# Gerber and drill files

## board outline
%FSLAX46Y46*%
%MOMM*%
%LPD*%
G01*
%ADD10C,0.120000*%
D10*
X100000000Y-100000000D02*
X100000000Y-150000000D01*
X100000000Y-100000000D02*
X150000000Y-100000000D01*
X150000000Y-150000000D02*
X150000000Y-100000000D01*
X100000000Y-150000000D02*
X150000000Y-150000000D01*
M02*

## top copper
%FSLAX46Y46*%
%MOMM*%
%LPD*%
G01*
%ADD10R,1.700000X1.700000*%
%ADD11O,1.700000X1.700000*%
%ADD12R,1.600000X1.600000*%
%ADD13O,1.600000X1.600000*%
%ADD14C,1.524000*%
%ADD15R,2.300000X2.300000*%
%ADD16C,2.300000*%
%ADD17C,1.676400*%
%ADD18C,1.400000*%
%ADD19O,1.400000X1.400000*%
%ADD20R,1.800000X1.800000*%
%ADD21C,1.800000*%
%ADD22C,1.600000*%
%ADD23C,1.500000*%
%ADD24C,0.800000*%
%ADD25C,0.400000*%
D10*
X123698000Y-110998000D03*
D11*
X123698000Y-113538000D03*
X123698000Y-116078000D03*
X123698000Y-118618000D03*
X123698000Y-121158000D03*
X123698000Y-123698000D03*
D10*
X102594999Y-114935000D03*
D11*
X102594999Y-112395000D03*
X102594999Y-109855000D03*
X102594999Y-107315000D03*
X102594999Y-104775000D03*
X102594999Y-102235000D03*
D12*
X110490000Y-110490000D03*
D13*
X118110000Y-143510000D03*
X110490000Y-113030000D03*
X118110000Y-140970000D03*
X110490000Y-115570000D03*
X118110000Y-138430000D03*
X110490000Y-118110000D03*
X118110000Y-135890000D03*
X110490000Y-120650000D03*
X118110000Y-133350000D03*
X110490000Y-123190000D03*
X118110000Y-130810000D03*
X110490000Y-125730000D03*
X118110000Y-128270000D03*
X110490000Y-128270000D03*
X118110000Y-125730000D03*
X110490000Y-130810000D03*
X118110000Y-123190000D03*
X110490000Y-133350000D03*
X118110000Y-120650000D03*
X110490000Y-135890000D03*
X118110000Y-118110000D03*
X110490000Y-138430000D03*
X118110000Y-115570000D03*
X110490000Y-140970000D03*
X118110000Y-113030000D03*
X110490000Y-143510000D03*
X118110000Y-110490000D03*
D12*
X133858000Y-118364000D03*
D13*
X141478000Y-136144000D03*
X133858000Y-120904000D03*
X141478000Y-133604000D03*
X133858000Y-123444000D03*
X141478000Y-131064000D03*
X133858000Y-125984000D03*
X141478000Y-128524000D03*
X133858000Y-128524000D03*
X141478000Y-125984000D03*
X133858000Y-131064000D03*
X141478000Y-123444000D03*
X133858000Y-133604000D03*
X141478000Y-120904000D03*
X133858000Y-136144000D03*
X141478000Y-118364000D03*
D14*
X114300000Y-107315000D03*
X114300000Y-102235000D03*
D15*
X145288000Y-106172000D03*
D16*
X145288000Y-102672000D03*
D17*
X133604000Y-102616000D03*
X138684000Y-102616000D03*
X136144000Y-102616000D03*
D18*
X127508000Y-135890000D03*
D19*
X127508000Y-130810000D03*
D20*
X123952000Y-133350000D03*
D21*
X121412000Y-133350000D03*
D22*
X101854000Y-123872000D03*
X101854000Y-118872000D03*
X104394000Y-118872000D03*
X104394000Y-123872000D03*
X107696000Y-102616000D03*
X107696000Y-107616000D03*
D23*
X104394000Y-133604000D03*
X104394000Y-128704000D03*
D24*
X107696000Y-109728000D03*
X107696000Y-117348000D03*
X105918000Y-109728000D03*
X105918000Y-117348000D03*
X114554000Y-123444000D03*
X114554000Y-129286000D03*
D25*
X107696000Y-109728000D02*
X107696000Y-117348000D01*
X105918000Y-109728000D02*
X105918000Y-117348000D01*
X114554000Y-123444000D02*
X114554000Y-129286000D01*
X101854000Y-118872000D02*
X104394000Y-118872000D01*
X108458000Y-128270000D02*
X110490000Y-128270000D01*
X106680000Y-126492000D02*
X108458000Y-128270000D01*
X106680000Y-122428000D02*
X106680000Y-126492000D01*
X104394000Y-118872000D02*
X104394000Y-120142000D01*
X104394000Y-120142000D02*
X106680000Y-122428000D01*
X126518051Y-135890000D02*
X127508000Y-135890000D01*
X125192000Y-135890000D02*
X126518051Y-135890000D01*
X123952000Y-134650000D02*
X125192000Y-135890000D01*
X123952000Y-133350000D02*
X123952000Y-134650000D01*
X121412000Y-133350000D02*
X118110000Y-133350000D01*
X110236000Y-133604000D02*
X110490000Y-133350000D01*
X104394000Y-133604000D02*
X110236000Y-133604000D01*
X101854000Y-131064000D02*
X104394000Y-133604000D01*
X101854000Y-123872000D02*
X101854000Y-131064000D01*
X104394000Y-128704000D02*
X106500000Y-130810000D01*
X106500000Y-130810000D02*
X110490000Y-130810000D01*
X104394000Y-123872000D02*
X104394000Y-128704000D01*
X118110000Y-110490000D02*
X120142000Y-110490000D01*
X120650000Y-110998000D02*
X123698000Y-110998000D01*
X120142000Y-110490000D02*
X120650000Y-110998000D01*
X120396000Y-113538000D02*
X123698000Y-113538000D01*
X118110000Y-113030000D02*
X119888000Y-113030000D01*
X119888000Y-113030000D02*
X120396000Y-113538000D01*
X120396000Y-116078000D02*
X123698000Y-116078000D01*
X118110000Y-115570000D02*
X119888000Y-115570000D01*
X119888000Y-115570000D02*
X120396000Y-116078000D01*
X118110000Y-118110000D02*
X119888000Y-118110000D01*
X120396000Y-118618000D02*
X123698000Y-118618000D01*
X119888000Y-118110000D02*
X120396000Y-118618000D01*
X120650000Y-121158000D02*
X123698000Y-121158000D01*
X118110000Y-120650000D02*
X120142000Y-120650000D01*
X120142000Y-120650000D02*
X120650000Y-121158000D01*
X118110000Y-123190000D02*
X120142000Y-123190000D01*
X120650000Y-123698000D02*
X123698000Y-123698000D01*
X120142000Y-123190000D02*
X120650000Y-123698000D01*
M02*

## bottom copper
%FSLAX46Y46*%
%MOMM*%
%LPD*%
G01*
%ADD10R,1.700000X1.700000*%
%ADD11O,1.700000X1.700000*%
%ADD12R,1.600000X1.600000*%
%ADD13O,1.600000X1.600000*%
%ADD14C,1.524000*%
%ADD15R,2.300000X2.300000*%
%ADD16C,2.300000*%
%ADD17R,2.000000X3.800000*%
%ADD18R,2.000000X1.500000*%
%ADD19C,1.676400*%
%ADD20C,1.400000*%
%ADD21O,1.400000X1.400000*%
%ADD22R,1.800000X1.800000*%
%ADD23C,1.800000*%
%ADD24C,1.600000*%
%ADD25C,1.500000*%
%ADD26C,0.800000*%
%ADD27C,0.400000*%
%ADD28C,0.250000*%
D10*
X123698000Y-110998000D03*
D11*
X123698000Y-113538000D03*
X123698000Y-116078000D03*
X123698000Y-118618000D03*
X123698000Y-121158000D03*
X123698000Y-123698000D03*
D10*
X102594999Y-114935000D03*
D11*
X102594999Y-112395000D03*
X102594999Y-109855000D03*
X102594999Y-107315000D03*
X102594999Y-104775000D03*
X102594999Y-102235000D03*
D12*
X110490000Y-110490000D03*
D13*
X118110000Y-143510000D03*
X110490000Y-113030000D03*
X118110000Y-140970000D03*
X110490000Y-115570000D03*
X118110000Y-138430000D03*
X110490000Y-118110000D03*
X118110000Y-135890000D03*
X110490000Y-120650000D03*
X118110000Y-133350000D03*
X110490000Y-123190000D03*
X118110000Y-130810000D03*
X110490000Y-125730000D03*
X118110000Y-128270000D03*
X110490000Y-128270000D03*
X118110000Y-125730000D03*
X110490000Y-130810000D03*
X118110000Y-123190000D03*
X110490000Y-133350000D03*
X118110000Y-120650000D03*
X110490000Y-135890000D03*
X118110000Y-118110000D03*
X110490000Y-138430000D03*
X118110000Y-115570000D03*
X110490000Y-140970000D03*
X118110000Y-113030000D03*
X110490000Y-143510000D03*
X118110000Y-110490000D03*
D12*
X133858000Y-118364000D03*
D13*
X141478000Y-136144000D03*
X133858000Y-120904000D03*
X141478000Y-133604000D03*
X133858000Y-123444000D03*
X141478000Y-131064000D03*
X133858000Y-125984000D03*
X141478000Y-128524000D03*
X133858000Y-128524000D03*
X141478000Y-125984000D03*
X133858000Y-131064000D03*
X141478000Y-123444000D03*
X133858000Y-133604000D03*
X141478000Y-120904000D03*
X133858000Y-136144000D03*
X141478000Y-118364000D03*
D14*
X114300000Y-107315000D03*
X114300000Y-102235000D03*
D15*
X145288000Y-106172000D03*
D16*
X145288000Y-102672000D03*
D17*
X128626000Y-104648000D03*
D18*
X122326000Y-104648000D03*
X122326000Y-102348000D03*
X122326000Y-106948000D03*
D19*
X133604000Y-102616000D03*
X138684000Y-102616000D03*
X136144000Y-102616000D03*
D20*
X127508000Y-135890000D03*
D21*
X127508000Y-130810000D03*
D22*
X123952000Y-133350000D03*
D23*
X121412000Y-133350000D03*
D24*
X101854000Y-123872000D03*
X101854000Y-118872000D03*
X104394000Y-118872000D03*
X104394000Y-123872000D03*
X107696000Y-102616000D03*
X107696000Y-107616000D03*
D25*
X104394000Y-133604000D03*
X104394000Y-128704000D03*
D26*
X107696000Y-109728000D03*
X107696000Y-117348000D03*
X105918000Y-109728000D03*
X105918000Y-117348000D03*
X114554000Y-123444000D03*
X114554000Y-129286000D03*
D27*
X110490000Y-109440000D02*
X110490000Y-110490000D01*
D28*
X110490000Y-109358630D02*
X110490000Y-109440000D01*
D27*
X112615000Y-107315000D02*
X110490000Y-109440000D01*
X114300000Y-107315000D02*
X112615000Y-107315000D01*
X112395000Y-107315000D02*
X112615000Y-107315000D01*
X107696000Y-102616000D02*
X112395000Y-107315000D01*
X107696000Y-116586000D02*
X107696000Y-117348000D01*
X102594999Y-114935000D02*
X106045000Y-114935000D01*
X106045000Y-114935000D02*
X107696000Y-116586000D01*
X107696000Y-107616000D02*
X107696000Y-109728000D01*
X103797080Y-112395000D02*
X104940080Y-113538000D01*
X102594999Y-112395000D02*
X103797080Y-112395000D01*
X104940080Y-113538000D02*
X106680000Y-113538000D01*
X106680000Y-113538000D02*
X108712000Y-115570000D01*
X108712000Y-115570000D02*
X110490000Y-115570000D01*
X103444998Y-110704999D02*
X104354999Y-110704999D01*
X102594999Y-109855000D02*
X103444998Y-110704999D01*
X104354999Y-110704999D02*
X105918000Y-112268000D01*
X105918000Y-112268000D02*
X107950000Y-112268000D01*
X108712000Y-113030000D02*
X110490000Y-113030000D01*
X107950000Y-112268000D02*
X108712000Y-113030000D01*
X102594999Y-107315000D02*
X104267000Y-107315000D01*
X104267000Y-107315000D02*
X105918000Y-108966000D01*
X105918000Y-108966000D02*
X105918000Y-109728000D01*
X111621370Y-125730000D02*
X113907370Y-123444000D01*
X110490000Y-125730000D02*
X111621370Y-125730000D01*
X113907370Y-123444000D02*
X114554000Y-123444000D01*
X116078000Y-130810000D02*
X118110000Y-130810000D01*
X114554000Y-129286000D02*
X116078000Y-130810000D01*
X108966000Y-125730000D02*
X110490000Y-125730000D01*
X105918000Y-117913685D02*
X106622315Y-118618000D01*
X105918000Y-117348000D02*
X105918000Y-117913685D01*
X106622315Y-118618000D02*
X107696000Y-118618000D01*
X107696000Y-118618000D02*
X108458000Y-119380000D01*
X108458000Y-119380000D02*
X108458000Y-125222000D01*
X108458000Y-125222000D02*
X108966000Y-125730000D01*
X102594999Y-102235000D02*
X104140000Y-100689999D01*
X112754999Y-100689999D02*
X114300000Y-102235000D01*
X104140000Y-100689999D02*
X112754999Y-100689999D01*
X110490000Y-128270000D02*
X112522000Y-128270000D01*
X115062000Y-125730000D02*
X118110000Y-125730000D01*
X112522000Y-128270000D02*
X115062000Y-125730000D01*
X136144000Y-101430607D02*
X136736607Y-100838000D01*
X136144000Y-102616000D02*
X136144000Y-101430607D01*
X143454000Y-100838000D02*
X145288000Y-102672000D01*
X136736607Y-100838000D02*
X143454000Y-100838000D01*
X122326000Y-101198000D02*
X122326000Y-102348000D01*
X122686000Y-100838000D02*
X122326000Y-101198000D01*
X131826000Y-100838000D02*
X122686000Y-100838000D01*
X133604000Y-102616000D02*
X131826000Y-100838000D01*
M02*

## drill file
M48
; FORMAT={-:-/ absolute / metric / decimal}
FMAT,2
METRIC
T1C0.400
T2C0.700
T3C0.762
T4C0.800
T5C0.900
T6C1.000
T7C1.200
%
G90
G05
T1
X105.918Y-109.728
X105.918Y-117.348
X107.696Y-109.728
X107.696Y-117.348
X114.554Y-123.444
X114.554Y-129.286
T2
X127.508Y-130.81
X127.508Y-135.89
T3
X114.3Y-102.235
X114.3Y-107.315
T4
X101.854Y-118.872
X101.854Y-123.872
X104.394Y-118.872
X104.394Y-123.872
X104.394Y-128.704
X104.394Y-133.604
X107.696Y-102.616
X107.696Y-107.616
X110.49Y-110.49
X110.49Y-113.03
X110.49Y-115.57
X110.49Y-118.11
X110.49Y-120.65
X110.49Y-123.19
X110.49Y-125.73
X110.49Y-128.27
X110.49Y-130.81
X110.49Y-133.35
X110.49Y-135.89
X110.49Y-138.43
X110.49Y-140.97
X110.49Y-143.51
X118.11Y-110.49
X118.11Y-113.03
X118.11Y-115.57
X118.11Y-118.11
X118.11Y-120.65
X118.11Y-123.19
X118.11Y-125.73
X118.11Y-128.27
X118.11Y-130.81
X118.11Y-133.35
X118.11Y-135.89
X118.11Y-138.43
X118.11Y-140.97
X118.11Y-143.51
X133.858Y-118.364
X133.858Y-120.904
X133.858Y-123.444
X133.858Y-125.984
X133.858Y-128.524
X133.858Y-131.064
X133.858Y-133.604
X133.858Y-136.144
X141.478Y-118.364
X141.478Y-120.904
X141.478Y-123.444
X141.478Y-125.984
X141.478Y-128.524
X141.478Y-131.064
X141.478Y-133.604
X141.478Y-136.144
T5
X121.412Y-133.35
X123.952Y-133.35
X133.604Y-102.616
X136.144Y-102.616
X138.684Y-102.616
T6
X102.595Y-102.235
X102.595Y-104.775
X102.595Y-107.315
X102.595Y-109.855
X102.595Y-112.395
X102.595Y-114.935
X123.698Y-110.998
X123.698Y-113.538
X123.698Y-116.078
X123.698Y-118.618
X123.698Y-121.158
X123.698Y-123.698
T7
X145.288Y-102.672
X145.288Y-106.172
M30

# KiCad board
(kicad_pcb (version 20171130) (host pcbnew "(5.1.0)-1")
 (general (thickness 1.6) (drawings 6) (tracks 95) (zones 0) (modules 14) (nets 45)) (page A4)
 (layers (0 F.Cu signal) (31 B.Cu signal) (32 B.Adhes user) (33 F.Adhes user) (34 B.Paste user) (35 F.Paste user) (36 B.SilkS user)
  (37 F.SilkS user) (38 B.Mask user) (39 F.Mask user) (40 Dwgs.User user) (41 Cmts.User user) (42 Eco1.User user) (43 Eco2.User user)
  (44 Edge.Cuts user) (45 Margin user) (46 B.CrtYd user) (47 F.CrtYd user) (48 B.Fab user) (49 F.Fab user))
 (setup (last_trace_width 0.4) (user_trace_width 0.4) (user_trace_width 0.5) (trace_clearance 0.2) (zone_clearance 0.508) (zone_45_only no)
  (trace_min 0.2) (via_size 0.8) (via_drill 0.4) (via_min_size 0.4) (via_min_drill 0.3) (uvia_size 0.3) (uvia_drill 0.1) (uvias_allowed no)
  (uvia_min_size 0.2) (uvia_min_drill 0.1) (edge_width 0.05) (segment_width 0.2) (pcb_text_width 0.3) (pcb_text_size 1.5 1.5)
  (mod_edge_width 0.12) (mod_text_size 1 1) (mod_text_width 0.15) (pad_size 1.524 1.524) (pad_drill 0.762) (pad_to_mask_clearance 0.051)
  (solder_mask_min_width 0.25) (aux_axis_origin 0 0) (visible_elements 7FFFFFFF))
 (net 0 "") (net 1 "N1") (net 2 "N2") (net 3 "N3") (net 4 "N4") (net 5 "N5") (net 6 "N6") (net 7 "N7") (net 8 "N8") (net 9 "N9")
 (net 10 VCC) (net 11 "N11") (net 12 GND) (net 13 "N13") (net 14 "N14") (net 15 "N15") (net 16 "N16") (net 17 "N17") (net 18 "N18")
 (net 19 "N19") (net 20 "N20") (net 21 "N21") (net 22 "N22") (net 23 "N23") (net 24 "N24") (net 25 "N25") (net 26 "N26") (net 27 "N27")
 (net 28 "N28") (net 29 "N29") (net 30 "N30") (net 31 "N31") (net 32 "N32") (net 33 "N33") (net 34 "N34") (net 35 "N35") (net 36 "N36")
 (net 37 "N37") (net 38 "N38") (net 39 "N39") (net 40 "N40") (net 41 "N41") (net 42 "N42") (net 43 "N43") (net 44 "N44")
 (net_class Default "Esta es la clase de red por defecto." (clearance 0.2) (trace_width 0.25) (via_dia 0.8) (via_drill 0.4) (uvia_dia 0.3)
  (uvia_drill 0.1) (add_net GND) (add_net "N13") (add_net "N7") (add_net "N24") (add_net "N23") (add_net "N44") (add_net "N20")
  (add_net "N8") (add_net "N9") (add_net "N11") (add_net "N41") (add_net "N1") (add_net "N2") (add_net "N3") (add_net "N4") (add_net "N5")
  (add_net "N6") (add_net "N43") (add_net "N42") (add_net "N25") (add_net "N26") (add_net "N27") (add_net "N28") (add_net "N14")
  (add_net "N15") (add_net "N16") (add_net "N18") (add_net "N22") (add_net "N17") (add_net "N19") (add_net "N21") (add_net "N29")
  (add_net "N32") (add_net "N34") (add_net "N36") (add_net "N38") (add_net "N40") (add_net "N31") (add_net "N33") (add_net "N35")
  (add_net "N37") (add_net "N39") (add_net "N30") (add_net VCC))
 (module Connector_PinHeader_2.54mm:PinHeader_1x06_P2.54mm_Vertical (layer F.Cu) (at 123.698 110.998)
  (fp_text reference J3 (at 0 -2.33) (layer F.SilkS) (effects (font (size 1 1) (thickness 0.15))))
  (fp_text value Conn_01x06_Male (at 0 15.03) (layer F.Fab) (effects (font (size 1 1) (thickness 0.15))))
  (pad 1 thru_hole rect (at 0 0) (size 1.7 1.7) (drill 1) (layers *.Cu *.Mask) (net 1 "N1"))
  (pad 2 thru_hole oval (at 0 2.54) (size 1.7 1.7) (drill 1) (layers *.Cu *.Mask) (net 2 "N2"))
  (pad 3 thru_hole oval (at 0 5.08) (size 1.7 1.7) (drill 1) (layers *.Cu *.Mask) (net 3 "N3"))
  (pad 4 thru_hole oval (at 0 7.62) (size 1.7 1.7) (drill 1) (layers *.Cu *.Mask) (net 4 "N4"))
  (pad 5 thru_hole oval (at 0 10.16) (size 1.7 1.7) (drill 1) (layers *.Cu *.Mask) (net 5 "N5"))
  (pad 6 thru_hole oval (at 0 12.7) (size 1.7 1.7) (drill 1) (layers *.Cu *.Mask) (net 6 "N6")))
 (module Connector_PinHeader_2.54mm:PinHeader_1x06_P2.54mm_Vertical (layer F.Cu) (at 102.594999 114.935 180)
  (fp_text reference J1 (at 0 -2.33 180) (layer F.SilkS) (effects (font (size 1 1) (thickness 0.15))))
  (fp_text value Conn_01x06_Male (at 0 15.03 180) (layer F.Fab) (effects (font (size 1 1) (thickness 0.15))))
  (pad 1 thru_hole rect (at 0 0 180) (size 1.7 1.7) (drill 1) (layers *.Cu *.Mask) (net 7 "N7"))
  (pad 2 thru_hole oval (at 0 2.54 180) (size 1.7 1.7) (drill 1) (layers *.Cu *.Mask) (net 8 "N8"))
  (pad 3 thru_hole oval (at 0 5.08 180) (size 1.7 1.7) (drill 1) (layers *.Cu *.Mask) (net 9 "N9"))
  (pad 4 thru_hole oval (at 0 7.62 180) (size 1.7 1.7) (drill 1) (layers *.Cu *.Mask) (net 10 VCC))
  (pad 5 thru_hole oval (at 0 10.16 180) (size 1.7 1.7) (drill 1) (layers *.Cu *.Mask) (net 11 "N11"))
  (pad 6 thru_hole oval (at 0 12.7 180) (size 1.7 1.7) (drill 1) (layers *.Cu *.Mask) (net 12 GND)))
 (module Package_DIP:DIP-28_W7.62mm (layer F.Cu) (at 110.49 110.49)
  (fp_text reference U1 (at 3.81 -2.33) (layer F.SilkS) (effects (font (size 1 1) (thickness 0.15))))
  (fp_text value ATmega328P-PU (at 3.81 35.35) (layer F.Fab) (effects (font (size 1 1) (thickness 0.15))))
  (pad 1 thru_hole rect (at 0 0) (size 1.6 1.6) (drill 0.8) (layers *.Cu *.Mask) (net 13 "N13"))
  (pad 15 thru_hole oval (at 7.62 33.02) (size 1.6 1.6) (drill 0.8) (layers *.Cu *.Mask) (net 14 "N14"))
  (pad 2 thru_hole oval (at 0 2.54) (size 1.6 1.6) (drill 0.8) (layers *.Cu *.Mask) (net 9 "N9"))
  (pad 16 thru_hole oval (at 7.62 30.48) (size 1.6 1.6) (drill 0.8) (layers *.Cu *.Mask) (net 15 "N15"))
  (pad 3 thru_hole oval (at 0 5.08) (size 1.6 1.6) (drill 0.8) (layers *.Cu *.Mask) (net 8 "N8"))
  (pad 17 thru_hole oval (at 7.62 27.94) (size 1.6 1.6) (drill 0.8) (layers *.Cu *.Mask) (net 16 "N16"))
  (pad 4 thru_hole oval (at 0 7.62) (size 1.6 1.6) (drill 0.8) (layers *.Cu *.Mask) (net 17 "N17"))
  (pad 18 thru_hole oval (at 7.62 25.4) (size 1.6 1.6) (drill 0.8) (layers *.Cu *.Mask) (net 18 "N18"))
  (pad 5 thru_hole oval (at 0 10.16) (size 1.6 1.6) (drill 0.8) (layers *.Cu *.Mask) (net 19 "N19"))
  (pad 19 thru_hole oval (at 7.62 22.86) (size 1.6 1.6) (drill 0.8) (layers *.Cu *.Mask) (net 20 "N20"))
  (pad 6 thru_hole oval (at 0 12.7) (size 1.6 1.6) (drill 0.8) (layers *.Cu *.Mask) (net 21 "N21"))
  (pad 20 thru_hole oval (at 7.62 20.32) (size 1.6 1.6) (drill 0.8) (layers *.Cu *.Mask) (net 10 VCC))
  (pad 7 thru_hole oval (at 0 15.24) (size 1.6 1.6) (drill 0.8) (layers *.Cu *.Mask) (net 10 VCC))
  (pad 21 thru_hole oval (at 7.62 17.78) (size 1.6 1.6) (drill 0.8) (layers *.Cu *.Mask) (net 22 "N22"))
  (pad 8 thru_hole oval (at 0 17.78) (size 1.6 1.6) (drill 0.8) (layers *.Cu *.Mask) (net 12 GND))
  (pad 22 thru_hole oval (at 7.62 15.24) (size 1.6 1.6) (drill 0.8) (layers *.Cu *.Mask) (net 12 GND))
  (pad 9 thru_hole oval (at 0 20.32) (size 1.6 1.6) (drill 0.8) (layers *.Cu *.Mask) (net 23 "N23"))
  (pad 23 thru_hole oval (at 7.62 12.7) (size 1.6 1.6) (drill 0.8) (layers *.Cu *.Mask) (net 6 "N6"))
  (pad 10 thru_hole oval (at 0 22.86) (size 1.6 1.6) (drill 0.8) (layers *.Cu *.Mask) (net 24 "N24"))
  (pad 24 thru_hole oval (at 7.62 10.16) (size 1.6 1.6) (drill 0.8) (layers *.Cu *.Mask) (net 5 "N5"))
  (pad 11 thru_hole oval (at 0 25.4) (size 1.6 1.6) (drill 0.8) (layers *.Cu *.Mask) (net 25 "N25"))
  (pad 25 thru_hole oval (at 7.62 7.62) (size 1.6 1.6) (drill 0.8) (layers *.Cu *.Mask) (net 4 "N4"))
  (pad 12 thru_hole oval (at 0 27.94) (size 1.6 1.6) (drill 0.8) (layers *.Cu *.Mask) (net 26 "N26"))
  (pad 26 thru_hole oval (at 7.62 5.08) (size 1.6 1.6) (drill 0.8) (layers *.Cu *.Mask) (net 3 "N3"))
  (pad 13 thru_hole oval (at 0 30.48) (size 1.6 1.6) (drill 0.8) (layers *.Cu *.Mask) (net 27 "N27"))
  (pad 27 thru_hole oval (at 7.62 2.54) (size 1.6 1.6) (drill 0.8) (layers *.Cu *.Mask) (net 2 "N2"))
  (pad 14 thru_hole oval (at 0 33.02) (size 1.6 1.6) (drill 0.8) (layers *.Cu *.Mask) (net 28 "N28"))
  (pad 28 thru_hole oval (at 7.62 0) (size 1.6 1.6) (drill 0.8) (layers *.Cu *.Mask) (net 1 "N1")))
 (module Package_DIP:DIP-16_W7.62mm (layer F.Cu) (at 133.858 118.364)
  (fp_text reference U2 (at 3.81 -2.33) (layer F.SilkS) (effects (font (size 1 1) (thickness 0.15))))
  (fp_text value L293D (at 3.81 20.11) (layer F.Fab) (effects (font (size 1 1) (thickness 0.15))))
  (pad 1 thru_hole rect (at 0 0) (size 1.6 1.6) (drill 0.8) (layers *.Cu *.Mask) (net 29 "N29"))
  (pad 9 thru_hole oval (at 7.62 17.78) (size 1.6 1.6) (drill 0.8) (layers *.Cu *.Mask) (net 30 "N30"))
  (pad 2 thru_hole oval (at 0 2.54) (size 1.6 1.6) (drill 0.8) (layers *.Cu *.Mask) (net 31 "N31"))
  (pad 10 thru_hole oval (at 7.62 15.24) (size 1.6 1.6) (drill 0.8) (layers *.Cu *.Mask) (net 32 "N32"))
  (pad 3 thru_hole oval (at 0 5.08) (size 1.6 1.6) (drill 0.8) (layers *.Cu *.Mask) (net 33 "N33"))
  (pad 11 thru_hole oval (at 7.62 12.7) (size 1.6 1.6) (drill 0.8) (layers *.Cu *.Mask) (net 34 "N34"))
  (pad 4 thru_hole oval (at 0 7.62) (size 1.6 1.6) (drill 0.8) (layers *.Cu *.Mask) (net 12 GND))
  (pad 12 thru_hole oval (at 7.62 10.16) (size 1.6 1.6) (drill 0.8) (layers *.Cu *.Mask) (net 12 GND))
  (pad 5 thru_hole oval (at 0 10.16) (size 1.6 1.6) (drill 0.8) (layers *.Cu *.Mask) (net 12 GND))
  (pad 13 thru_hole oval (at 7.62 7.62) (size 1.6 1.6) (drill 0.8) (layers *.Cu *.Mask) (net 12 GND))
  (pad 6 thru_hole oval (at 0 12.7) (size 1.6 1.6) (drill 0.8) (layers *.Cu *.Mask) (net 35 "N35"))
  (pad 14 thru_hole oval (at 7.62 5.08) (size 1.6 1.6) (drill 0.8) (layers *.Cu *.Mask) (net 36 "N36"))
  (pad 7 thru_hole oval (at 0 15.24) (size 1.6 1.6) (drill 0.8) (layers *.Cu *.Mask) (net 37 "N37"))
  (pad 15 thru_hole oval (at 7.62 2.54) (size 1.6 1.6) (drill 0.8) (layers *.Cu *.Mask) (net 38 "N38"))
  (pad 8 thru_hole oval (at 0 17.78) (size 1.6 1.6) (drill 0.8) (layers *.Cu *.Mask) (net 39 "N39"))
  (pad 16 thru_hole oval (at 7.62 0) (size 1.6 1.6) (drill 0.8) (layers *.Cu *.Mask) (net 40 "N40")))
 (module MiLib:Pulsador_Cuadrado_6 (layer F.Cu) (at 111.76 104.775 90)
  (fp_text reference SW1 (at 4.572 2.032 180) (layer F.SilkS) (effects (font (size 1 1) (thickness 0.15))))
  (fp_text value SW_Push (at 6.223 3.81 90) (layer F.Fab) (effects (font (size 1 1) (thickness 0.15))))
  (pad 1 thru_hole circle (at -2.54 2.54 90) (size 1.524 1.524) (drill 0.762) (layers *.Cu *.Mask) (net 13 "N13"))
  (pad 2 thru_hole circle (at 2.54 2.54 90) (size 1.524 1.524) (drill 0.762) (layers *.Cu *.Mask) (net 12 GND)))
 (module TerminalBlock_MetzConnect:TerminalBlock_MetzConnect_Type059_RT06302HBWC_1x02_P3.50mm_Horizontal (layer F.Cu)
  (at 145.288 106.172 90)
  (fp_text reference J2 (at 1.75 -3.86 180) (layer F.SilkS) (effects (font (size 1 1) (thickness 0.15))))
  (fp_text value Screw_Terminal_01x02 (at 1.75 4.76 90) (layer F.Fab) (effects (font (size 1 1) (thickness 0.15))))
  (pad 1 thru_hole rect (at 0 0 90) (size 2.3 2.3) (drill 1.2) (layers *.Cu *.Mask) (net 12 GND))
  (pad 2 thru_hole circle (at 3.5 0 90) (size 2.3 2.3) (drill 1.2) (layers *.Cu *.Mask) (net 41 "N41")))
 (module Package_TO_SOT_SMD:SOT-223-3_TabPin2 (layer B.Cu) (at 125.476 104.648)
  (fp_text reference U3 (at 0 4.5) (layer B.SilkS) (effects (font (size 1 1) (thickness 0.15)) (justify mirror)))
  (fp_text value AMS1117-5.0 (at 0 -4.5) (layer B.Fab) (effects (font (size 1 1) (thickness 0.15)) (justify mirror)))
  (pad 2 smd rect (at 3.15 0) (size 2 3.8) (layers B.Cu B.Paste B.Mask) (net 10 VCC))
  (pad 2 smd rect (at -3.15 0) (size 2 1.5) (layers B.Cu B.Paste B.Mask) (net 10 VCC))
  (pad 3 smd rect (at -3.15 -2.3) (size 2 1.5) (layers B.Cu B.Paste B.Mask) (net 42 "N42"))
  (pad 1 smd rect (at -3.15 2.3) (size 2 1.5) (layers B.Cu B.Paste B.Mask) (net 12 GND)))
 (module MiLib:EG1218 (layer F.Cu) (at 136.144 102.616 180)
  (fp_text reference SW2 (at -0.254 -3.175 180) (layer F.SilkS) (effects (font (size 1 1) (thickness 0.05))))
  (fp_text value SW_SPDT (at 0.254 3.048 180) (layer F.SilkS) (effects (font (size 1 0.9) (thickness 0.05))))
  (pad 3 thru_hole circle (at 2.54 0 180) (size 1.6764 1.6764) (drill 0.9) (layers *.Cu *.Mask) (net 42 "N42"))
  (pad 1 thru_hole circle (at -2.54 0 180) (size 1.6764 1.6764) (drill 0.9) (layers *.Cu *.Mask) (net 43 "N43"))
  (pad 2 thru_hole circle (at 0 0 180) (size 1.6764 1.6764) (drill 0.9) (layers *.Cu *.Mask) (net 41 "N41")))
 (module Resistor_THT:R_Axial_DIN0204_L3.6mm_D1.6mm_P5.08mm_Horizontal (layer F.Cu) (at 127.508 135.89 90)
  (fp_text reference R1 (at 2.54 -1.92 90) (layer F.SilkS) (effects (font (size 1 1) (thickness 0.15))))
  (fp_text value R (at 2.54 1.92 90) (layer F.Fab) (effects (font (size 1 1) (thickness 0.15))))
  (pad 1 thru_hole circle (at 0 0 90) (size 1.4 1.4) (drill 0.7) (layers *.Cu *.Mask) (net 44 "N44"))
  (pad 2 thru_hole oval (at 5.08 0 90) (size 1.4 1.4) (drill 0.7) (layers *.Cu *.Mask) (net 12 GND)))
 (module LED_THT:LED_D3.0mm (layer F.Cu) (at 123.952 133.35 180)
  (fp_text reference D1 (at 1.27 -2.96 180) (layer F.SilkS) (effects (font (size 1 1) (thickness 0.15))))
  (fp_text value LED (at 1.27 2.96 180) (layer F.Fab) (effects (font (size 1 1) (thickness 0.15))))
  (pad 1 thru_hole rect (at 0 0 180) (size 1.8 1.8) (drill 0.9) (layers *.Cu *.Mask) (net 44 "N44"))
  (pad 2 thru_hole circle (at 2.54 0 180) (size 1.8 1.8) (drill 0.9) (layers *.Cu *.Mask) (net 20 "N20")))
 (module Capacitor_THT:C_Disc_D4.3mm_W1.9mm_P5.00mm (layer F.Cu) (at 101.854 123.872 90)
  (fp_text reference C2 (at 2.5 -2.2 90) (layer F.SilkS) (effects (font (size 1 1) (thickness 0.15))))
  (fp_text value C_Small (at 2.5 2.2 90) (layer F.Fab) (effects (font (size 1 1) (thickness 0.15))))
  (pad 1 thru_hole circle (at 0 0 90) (size 1.6 1.6) (drill 0.8) (layers *.Cu *.Mask) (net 24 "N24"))
  (pad 2 thru_hole circle (at 5 0 90) (size 1.6 1.6) (drill 0.8) (layers *.Cu *.Mask) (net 12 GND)))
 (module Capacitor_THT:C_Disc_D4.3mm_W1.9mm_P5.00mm (layer F.Cu) (at 104.394 123.872 90)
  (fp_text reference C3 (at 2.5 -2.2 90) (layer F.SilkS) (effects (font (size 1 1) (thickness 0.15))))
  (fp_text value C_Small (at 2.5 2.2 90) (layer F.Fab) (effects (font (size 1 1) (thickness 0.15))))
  (pad 2 thru_hole circle (at 5 0 90) (size 1.6 1.6) (drill 0.8) (layers *.Cu *.Mask) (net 12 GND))
  (pad 1 thru_hole circle (at 0 0 90) (size 1.6 1.6) (drill 0.8) (layers *.Cu *.Mask) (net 23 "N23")))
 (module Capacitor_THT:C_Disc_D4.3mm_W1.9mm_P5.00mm (layer F.Cu) (at 107.696 102.616 270)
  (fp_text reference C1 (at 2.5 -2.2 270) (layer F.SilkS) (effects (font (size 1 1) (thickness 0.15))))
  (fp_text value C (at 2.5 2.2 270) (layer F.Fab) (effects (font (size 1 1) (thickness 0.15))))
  (pad 1 thru_hole circle (at 0 0 270) (size 1.6 1.6) (drill 0.8) (layers *.Cu *.Mask) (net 13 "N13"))
  (pad 2 thru_hole circle (at 5 0 270) (size 1.6 1.6) (drill 0.8) (layers *.Cu *.Mask) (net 7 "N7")))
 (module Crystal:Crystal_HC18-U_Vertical (layer F.Cu) (at 104.394 133.604 90)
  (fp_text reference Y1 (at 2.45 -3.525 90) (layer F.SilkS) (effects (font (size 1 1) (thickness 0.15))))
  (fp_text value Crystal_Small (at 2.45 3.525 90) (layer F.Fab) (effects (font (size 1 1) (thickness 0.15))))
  (pad 1 thru_hole circle (at 0 0 90) (size 1.5 1.5) (drill 0.8) (layers *.Cu *.Mask) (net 24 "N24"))
  (pad 2 thru_hole circle (at 4.9 0 90) (size 1.5 1.5) (drill 0.8) (layers *.Cu *.Mask) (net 23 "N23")))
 (gr_line (start 100 100) (end 100 150) (layer Edge.Cuts) (width 0.12))
 (gr_line (start 100 100) (end 150 100) (layer Edge.Cuts) (width 0.12))
 (gr_line (start 150 150) (end 150 100) (layer Edge.Cuts) (width 0.12))
 (gr_line (start 100 150) (end 150 150) (layer Edge.Cuts) (width 0.12))
 (segment (start 110.49 109.44) (end 110.49 110.49) (width 0.4) (layer B.Cu) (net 13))
 (segment (start 110.49 109.35863) (end 110.49 109.44) (width 0.25) (layer B.Cu) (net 13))
 (segment (start 112.615 107.315) (end 110.49 109.44) (width 0.4) (layer B.Cu) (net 13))
 (segment (start 114.3 107.315) (end 112.615 107.315) (width 0.4) (layer B.Cu) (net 13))
 (segment (start 112.395 107.315) (end 112.615 107.315) (width 0.4) (layer B.Cu) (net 13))
 (segment (start 107.696 102.616) (end 112.395 107.315) (width 0.4) (layer B.Cu) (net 13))
 (via (at 107.696 109.728) (size 0.8) (drill 0.4) (layers F.Cu B.Cu) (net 7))
 (via (at 107.696 117.348) (size 0.8) (drill 0.4) (layers F.Cu B.Cu) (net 7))
 (segment (start 107.696 109.728) (end 107.696 117.348) (width 0.4) (layer F.Cu) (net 7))
 (segment (start 107.696 116.586) (end 107.696 117.348) (width 0.4) (layer B.Cu) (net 7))
 (segment (start 102.594999 114.935) (end 106.045 114.935) (width 0.4) (layer B.Cu) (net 7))
 (segment (start 106.045 114.935) (end 107.696 116.586) (width 0.4) (layer B.Cu) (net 7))
 (segment (start 107.696 107.616) (end 107.696 109.728) (width 0.4) (layer B.Cu) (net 7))
 (segment (start 103.79708 112.395) (end 104.94008 113.538) (width 0.4) (layer B.Cu) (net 8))
 (segment (start 102.594999 112.395) (end 103.79708 112.395) (width 0.4) (layer B.Cu) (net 8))
 (segment (start 104.94008 113.538) (end 106.68 113.538) (width 0.4) (layer B.Cu) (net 8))
 (segment (start 106.68 113.538) (end 108.712 115.57) (width 0.4) (layer B.Cu) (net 8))
 (segment (start 108.712 115.57) (end 110.49 115.57) (width 0.4) (layer B.Cu) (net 8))
 (segment (start 103.444998 110.704999) (end 104.354999 110.704999) (width 0.4) (layer B.Cu) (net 9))
 (segment (start 102.594999 109.855) (end 103.444998 110.704999) (width 0.4) (layer B.Cu) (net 9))
 (segment (start 104.354999 110.704999) (end 105.918 112.268) (width 0.4) (layer B.Cu) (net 9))
 (segment (start 105.918 112.268) (end 107.95 112.268) (width 0.4) (layer B.Cu) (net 9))
 (segment (start 108.712 113.03) (end 110.49 113.03) (width 0.4) (layer B.Cu) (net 9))
 (segment (start 107.95 112.268) (end 108.712 113.03) (width 0.4) (layer B.Cu) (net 9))
 (segment (start 102.594999 107.315) (end 104.267 107.315) (width 0.4) (layer B.Cu) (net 10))
 (segment (start 104.267 107.315) (end 105.918 108.966) (width 0.4) (layer B.Cu) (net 10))
 (via (at 105.918 109.728) (size 0.8) (drill 0.4) (layers F.Cu B.Cu) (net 10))
 (segment (start 105.918 108.966) (end 105.918 109.728) (width 0.4) (layer B.Cu) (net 10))
 (segment (start 105.918 109.728) (end 105.918 117.348) (width 0.4) (layer F.Cu) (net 10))
 (via (at 105.918 117.348) (size 0.8) (drill 0.4) (layers F.Cu B.Cu) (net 10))
 (segment (start 111.62137 125.73) (end 113.90737 123.444) (width 0.4) (layer B.Cu) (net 10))
 (segment (start 110.49 125.73) (end 111.62137 125.73) (width 0.4) (layer B.Cu) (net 10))
 (via (at 114.554 123.444) (size 0.8) (drill 0.4) (layers F.Cu B.Cu) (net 10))
 (segment (start 113.90737 123.444) (end 114.554 123.444) (width 0.4) (layer B.Cu) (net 10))
 (segment (start 114.554 123.444) (end 114.554 129.286) (width 0.4) (layer F.Cu) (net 10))
 (via (at 114.554 129.286) (size 0.8) (drill 0.4) (layers F.Cu B.Cu) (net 10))
 (segment (start 116.078 130.81) (end 118.11 130.81) (width 0.4) (layer B.Cu) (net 10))
 (segment (start 114.554 129.286) (end 116.078 130.81) (width 0.4) (layer B.Cu) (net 10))
 (segment (start 108.966 125.73) (end 110.49 125.73) (width 0.4) (layer B.Cu) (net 10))
 (segment (start 105.918 117.913685) (end 106.622315 118.618) (width 0.4) (layer B.Cu) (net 10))
 (segment (start 105.918 117.348) (end 105.918 117.913685) (width 0.4) (layer B.Cu) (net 10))
 (segment (start 106.622315 118.618) (end 107.696 118.618) (width 0.4) (layer B.Cu) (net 10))
 (segment (start 107.696 118.618) (end 108.458 119.38) (width 0.4) (layer B.Cu) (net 10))
 (segment (start 108.458 119.38) (end 108.458 125.222) (width 0.4) (layer B.Cu) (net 10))
 (segment (start 108.458 125.222) (end 108.966 125.73) (width 0.4) (layer B.Cu) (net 10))
 (segment (start 102.594999 102.235) (end 104.14 100.689999) (width 0.4) (layer B.Cu) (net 12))
 (segment (start 112.754999 100.689999) (end 114.3 102.235) (width 0.4) (layer B.Cu) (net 12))
 (segment (start 104.14 100.689999) (end 112.754999 100.689999) (width 0.4) (layer B.Cu) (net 12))
 (segment (start 110.49 128.27) (end 112.522 128.27) (width 0.4) (layer B.Cu) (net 12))
 (segment (start 115.062 125.73) (end 118.11 125.73) (width 0.4) (layer B.Cu) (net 12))
 (segment (start 112.522 128.27) (end 115.062 125.73) (width 0.4) (layer B.Cu) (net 12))
 (segment (start 101.854 118.872) (end 104.394 118.872) (width 0.4) (layer F.Cu) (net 12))
 (segment (start 108.458 128.27) (end 110.49 128.27) (width 0.4) (layer F.Cu) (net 12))
 (segment (start 106.68 126.492) (end 108.458 128.27) (width 0.4) (layer F.Cu) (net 12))
 (segment (start 106.68 122.428) (end 106.68 126.492) (width 0.4) (layer F.Cu) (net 12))
 (segment (start 104.394 118.872) (end 104.394 120.142) (width 0.4) (layer F.Cu) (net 12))
 (segment (start 104.394 120.142) (end 106.68 122.428) (width 0.4) (layer F.Cu) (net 12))
 (segment (start 136.144 101.430607) (end 136.736607 100.838) (width 0.4) (layer B.Cu) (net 41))
 (segment (start 136.144 102.616) (end 136.144 101.430607) (width 0.4) (layer B.Cu) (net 41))
 (segment (start 143.454 100.838) (end 145.288 102.672) (width 0.4) (layer B.Cu) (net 41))
 (segment (start 136.736607 100.838) (end 143.454 100.838) (width 0.4) (layer B.Cu) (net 41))
 (segment (start 122.326 101.198) (end 122.326 102.348) (width 0.4) (layer B.Cu) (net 42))
 (segment (start 122.686 100.838) (end 122.326 101.198) (width 0.4) (layer B.Cu) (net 42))
 (segment (start 131.826 100.838) (end 122.686 100.838) (width 0.4) (layer B.Cu) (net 42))
 (segment (start 133.604 102.616) (end 131.826 100.838) (width 0.4) (layer B.Cu) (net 42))
 (segment (start 126.518051 135.89) (end 127.508 135.89) (width 0.4) (layer F.Cu) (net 44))
 (segment (start 125.192 135.89) (end 126.518051 135.89) (width 0.4) (layer F.Cu) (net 44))
 (segment (start 123.952 134.65) (end 125.192 135.89) (width 0.4) (layer F.Cu) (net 44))
 (segment (start 123.952 133.35) (end 123.952 134.65) (width 0.4) (layer F.Cu) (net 44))
 (segment (start 121.412 133.35) (end 118.11 133.35) (width 0.4) (layer F.Cu) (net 20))
 (segment (start 110.236 133.604) (end 110.49 133.35) (width 0.4) (layer F.Cu) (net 24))
 (segment (start 104.394 133.604) (end 110.236 133.604) (width 0.4) (layer F.Cu) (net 24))
 (segment (start 101.854 131.064) (end 104.394 133.604) (width 0.4) (layer F.Cu) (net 24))
 (segment (start 101.854 123.872) (end 101.854 131.064) (width 0.4) (layer F.Cu) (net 24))
 (segment (start 104.394 128.704) (end 106.5 130.81) (width 0.4) (layer F.Cu) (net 23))
 (segment (start 106.5 130.81) (end 110.49 130.81) (width 0.4) (layer F.Cu) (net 23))
 (segment (start 104.394 123.872) (end 104.394 128.704) (width 0.4) (layer F.Cu) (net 23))
 (segment (start 118.11 110.49) (end 120.142 110.49) (width 0.4) (layer F.Cu) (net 1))
 (segment (start 120.65 110.998) (end 123.698 110.998) (width 0.4) (layer F.Cu) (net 1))
 (segment (start 120.142 110.49) (end 120.65 110.998) (width 0.4) (layer F.Cu) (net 1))
 (segment (start 120.396 113.538) (end 123.698 113.538) (width 0.4) (layer F.Cu) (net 2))
 (segment (start 118.11 113.03) (end 119.888 113.03) (width 0.4) (layer F.Cu) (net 2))
 (segment (start 119.888 113.03) (end 120.396 113.538) (width 0.4) (layer F.Cu) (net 2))
 (segment (start 120.396 116.078) (end 123.698 116.078) (width 0.4) (layer F.Cu) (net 3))
 (segment (start 118.11 115.57) (end 119.888 115.57) (width 0.4) (layer F.Cu) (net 3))
 (segment (start 119.888 115.57) (end 120.396 116.078) (width 0.4) (layer F.Cu) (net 3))
 (segment (start 118.11 118.11) (end 119.888 118.11) (width 0.4) (layer F.Cu) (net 4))
 (segment (start 120.396 118.618) (end 123.698 118.618) (width 0.4) (layer F.Cu) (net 4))
 (segment (start 119.888 118.11) (end 120.396 118.618) (width 0.4) (layer F.Cu) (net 4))
 (segment (start 120.65 121.158) (end 123.698 121.158) (width 0.4) (layer F.Cu) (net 5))
 (segment (start 118.11 120.65) (end 120.142 120.65) (width 0.4) (layer F.Cu) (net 5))
 (segment (start 120.142 120.65) (end 120.65 121.158) (width 0.4) (layer F.Cu) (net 5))
 (segment (start 118.11 123.19) (end 120.142 123.19) (width 0.4) (layer F.Cu) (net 6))
 (segment (start 120.65 123.698) (end 123.698 123.698) (width 0.4) (layer F.Cu) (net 6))
 (segment (start 120.142 123.19) (end 120.65 123.698) (width 0.4) (layer F.Cu) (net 6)))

